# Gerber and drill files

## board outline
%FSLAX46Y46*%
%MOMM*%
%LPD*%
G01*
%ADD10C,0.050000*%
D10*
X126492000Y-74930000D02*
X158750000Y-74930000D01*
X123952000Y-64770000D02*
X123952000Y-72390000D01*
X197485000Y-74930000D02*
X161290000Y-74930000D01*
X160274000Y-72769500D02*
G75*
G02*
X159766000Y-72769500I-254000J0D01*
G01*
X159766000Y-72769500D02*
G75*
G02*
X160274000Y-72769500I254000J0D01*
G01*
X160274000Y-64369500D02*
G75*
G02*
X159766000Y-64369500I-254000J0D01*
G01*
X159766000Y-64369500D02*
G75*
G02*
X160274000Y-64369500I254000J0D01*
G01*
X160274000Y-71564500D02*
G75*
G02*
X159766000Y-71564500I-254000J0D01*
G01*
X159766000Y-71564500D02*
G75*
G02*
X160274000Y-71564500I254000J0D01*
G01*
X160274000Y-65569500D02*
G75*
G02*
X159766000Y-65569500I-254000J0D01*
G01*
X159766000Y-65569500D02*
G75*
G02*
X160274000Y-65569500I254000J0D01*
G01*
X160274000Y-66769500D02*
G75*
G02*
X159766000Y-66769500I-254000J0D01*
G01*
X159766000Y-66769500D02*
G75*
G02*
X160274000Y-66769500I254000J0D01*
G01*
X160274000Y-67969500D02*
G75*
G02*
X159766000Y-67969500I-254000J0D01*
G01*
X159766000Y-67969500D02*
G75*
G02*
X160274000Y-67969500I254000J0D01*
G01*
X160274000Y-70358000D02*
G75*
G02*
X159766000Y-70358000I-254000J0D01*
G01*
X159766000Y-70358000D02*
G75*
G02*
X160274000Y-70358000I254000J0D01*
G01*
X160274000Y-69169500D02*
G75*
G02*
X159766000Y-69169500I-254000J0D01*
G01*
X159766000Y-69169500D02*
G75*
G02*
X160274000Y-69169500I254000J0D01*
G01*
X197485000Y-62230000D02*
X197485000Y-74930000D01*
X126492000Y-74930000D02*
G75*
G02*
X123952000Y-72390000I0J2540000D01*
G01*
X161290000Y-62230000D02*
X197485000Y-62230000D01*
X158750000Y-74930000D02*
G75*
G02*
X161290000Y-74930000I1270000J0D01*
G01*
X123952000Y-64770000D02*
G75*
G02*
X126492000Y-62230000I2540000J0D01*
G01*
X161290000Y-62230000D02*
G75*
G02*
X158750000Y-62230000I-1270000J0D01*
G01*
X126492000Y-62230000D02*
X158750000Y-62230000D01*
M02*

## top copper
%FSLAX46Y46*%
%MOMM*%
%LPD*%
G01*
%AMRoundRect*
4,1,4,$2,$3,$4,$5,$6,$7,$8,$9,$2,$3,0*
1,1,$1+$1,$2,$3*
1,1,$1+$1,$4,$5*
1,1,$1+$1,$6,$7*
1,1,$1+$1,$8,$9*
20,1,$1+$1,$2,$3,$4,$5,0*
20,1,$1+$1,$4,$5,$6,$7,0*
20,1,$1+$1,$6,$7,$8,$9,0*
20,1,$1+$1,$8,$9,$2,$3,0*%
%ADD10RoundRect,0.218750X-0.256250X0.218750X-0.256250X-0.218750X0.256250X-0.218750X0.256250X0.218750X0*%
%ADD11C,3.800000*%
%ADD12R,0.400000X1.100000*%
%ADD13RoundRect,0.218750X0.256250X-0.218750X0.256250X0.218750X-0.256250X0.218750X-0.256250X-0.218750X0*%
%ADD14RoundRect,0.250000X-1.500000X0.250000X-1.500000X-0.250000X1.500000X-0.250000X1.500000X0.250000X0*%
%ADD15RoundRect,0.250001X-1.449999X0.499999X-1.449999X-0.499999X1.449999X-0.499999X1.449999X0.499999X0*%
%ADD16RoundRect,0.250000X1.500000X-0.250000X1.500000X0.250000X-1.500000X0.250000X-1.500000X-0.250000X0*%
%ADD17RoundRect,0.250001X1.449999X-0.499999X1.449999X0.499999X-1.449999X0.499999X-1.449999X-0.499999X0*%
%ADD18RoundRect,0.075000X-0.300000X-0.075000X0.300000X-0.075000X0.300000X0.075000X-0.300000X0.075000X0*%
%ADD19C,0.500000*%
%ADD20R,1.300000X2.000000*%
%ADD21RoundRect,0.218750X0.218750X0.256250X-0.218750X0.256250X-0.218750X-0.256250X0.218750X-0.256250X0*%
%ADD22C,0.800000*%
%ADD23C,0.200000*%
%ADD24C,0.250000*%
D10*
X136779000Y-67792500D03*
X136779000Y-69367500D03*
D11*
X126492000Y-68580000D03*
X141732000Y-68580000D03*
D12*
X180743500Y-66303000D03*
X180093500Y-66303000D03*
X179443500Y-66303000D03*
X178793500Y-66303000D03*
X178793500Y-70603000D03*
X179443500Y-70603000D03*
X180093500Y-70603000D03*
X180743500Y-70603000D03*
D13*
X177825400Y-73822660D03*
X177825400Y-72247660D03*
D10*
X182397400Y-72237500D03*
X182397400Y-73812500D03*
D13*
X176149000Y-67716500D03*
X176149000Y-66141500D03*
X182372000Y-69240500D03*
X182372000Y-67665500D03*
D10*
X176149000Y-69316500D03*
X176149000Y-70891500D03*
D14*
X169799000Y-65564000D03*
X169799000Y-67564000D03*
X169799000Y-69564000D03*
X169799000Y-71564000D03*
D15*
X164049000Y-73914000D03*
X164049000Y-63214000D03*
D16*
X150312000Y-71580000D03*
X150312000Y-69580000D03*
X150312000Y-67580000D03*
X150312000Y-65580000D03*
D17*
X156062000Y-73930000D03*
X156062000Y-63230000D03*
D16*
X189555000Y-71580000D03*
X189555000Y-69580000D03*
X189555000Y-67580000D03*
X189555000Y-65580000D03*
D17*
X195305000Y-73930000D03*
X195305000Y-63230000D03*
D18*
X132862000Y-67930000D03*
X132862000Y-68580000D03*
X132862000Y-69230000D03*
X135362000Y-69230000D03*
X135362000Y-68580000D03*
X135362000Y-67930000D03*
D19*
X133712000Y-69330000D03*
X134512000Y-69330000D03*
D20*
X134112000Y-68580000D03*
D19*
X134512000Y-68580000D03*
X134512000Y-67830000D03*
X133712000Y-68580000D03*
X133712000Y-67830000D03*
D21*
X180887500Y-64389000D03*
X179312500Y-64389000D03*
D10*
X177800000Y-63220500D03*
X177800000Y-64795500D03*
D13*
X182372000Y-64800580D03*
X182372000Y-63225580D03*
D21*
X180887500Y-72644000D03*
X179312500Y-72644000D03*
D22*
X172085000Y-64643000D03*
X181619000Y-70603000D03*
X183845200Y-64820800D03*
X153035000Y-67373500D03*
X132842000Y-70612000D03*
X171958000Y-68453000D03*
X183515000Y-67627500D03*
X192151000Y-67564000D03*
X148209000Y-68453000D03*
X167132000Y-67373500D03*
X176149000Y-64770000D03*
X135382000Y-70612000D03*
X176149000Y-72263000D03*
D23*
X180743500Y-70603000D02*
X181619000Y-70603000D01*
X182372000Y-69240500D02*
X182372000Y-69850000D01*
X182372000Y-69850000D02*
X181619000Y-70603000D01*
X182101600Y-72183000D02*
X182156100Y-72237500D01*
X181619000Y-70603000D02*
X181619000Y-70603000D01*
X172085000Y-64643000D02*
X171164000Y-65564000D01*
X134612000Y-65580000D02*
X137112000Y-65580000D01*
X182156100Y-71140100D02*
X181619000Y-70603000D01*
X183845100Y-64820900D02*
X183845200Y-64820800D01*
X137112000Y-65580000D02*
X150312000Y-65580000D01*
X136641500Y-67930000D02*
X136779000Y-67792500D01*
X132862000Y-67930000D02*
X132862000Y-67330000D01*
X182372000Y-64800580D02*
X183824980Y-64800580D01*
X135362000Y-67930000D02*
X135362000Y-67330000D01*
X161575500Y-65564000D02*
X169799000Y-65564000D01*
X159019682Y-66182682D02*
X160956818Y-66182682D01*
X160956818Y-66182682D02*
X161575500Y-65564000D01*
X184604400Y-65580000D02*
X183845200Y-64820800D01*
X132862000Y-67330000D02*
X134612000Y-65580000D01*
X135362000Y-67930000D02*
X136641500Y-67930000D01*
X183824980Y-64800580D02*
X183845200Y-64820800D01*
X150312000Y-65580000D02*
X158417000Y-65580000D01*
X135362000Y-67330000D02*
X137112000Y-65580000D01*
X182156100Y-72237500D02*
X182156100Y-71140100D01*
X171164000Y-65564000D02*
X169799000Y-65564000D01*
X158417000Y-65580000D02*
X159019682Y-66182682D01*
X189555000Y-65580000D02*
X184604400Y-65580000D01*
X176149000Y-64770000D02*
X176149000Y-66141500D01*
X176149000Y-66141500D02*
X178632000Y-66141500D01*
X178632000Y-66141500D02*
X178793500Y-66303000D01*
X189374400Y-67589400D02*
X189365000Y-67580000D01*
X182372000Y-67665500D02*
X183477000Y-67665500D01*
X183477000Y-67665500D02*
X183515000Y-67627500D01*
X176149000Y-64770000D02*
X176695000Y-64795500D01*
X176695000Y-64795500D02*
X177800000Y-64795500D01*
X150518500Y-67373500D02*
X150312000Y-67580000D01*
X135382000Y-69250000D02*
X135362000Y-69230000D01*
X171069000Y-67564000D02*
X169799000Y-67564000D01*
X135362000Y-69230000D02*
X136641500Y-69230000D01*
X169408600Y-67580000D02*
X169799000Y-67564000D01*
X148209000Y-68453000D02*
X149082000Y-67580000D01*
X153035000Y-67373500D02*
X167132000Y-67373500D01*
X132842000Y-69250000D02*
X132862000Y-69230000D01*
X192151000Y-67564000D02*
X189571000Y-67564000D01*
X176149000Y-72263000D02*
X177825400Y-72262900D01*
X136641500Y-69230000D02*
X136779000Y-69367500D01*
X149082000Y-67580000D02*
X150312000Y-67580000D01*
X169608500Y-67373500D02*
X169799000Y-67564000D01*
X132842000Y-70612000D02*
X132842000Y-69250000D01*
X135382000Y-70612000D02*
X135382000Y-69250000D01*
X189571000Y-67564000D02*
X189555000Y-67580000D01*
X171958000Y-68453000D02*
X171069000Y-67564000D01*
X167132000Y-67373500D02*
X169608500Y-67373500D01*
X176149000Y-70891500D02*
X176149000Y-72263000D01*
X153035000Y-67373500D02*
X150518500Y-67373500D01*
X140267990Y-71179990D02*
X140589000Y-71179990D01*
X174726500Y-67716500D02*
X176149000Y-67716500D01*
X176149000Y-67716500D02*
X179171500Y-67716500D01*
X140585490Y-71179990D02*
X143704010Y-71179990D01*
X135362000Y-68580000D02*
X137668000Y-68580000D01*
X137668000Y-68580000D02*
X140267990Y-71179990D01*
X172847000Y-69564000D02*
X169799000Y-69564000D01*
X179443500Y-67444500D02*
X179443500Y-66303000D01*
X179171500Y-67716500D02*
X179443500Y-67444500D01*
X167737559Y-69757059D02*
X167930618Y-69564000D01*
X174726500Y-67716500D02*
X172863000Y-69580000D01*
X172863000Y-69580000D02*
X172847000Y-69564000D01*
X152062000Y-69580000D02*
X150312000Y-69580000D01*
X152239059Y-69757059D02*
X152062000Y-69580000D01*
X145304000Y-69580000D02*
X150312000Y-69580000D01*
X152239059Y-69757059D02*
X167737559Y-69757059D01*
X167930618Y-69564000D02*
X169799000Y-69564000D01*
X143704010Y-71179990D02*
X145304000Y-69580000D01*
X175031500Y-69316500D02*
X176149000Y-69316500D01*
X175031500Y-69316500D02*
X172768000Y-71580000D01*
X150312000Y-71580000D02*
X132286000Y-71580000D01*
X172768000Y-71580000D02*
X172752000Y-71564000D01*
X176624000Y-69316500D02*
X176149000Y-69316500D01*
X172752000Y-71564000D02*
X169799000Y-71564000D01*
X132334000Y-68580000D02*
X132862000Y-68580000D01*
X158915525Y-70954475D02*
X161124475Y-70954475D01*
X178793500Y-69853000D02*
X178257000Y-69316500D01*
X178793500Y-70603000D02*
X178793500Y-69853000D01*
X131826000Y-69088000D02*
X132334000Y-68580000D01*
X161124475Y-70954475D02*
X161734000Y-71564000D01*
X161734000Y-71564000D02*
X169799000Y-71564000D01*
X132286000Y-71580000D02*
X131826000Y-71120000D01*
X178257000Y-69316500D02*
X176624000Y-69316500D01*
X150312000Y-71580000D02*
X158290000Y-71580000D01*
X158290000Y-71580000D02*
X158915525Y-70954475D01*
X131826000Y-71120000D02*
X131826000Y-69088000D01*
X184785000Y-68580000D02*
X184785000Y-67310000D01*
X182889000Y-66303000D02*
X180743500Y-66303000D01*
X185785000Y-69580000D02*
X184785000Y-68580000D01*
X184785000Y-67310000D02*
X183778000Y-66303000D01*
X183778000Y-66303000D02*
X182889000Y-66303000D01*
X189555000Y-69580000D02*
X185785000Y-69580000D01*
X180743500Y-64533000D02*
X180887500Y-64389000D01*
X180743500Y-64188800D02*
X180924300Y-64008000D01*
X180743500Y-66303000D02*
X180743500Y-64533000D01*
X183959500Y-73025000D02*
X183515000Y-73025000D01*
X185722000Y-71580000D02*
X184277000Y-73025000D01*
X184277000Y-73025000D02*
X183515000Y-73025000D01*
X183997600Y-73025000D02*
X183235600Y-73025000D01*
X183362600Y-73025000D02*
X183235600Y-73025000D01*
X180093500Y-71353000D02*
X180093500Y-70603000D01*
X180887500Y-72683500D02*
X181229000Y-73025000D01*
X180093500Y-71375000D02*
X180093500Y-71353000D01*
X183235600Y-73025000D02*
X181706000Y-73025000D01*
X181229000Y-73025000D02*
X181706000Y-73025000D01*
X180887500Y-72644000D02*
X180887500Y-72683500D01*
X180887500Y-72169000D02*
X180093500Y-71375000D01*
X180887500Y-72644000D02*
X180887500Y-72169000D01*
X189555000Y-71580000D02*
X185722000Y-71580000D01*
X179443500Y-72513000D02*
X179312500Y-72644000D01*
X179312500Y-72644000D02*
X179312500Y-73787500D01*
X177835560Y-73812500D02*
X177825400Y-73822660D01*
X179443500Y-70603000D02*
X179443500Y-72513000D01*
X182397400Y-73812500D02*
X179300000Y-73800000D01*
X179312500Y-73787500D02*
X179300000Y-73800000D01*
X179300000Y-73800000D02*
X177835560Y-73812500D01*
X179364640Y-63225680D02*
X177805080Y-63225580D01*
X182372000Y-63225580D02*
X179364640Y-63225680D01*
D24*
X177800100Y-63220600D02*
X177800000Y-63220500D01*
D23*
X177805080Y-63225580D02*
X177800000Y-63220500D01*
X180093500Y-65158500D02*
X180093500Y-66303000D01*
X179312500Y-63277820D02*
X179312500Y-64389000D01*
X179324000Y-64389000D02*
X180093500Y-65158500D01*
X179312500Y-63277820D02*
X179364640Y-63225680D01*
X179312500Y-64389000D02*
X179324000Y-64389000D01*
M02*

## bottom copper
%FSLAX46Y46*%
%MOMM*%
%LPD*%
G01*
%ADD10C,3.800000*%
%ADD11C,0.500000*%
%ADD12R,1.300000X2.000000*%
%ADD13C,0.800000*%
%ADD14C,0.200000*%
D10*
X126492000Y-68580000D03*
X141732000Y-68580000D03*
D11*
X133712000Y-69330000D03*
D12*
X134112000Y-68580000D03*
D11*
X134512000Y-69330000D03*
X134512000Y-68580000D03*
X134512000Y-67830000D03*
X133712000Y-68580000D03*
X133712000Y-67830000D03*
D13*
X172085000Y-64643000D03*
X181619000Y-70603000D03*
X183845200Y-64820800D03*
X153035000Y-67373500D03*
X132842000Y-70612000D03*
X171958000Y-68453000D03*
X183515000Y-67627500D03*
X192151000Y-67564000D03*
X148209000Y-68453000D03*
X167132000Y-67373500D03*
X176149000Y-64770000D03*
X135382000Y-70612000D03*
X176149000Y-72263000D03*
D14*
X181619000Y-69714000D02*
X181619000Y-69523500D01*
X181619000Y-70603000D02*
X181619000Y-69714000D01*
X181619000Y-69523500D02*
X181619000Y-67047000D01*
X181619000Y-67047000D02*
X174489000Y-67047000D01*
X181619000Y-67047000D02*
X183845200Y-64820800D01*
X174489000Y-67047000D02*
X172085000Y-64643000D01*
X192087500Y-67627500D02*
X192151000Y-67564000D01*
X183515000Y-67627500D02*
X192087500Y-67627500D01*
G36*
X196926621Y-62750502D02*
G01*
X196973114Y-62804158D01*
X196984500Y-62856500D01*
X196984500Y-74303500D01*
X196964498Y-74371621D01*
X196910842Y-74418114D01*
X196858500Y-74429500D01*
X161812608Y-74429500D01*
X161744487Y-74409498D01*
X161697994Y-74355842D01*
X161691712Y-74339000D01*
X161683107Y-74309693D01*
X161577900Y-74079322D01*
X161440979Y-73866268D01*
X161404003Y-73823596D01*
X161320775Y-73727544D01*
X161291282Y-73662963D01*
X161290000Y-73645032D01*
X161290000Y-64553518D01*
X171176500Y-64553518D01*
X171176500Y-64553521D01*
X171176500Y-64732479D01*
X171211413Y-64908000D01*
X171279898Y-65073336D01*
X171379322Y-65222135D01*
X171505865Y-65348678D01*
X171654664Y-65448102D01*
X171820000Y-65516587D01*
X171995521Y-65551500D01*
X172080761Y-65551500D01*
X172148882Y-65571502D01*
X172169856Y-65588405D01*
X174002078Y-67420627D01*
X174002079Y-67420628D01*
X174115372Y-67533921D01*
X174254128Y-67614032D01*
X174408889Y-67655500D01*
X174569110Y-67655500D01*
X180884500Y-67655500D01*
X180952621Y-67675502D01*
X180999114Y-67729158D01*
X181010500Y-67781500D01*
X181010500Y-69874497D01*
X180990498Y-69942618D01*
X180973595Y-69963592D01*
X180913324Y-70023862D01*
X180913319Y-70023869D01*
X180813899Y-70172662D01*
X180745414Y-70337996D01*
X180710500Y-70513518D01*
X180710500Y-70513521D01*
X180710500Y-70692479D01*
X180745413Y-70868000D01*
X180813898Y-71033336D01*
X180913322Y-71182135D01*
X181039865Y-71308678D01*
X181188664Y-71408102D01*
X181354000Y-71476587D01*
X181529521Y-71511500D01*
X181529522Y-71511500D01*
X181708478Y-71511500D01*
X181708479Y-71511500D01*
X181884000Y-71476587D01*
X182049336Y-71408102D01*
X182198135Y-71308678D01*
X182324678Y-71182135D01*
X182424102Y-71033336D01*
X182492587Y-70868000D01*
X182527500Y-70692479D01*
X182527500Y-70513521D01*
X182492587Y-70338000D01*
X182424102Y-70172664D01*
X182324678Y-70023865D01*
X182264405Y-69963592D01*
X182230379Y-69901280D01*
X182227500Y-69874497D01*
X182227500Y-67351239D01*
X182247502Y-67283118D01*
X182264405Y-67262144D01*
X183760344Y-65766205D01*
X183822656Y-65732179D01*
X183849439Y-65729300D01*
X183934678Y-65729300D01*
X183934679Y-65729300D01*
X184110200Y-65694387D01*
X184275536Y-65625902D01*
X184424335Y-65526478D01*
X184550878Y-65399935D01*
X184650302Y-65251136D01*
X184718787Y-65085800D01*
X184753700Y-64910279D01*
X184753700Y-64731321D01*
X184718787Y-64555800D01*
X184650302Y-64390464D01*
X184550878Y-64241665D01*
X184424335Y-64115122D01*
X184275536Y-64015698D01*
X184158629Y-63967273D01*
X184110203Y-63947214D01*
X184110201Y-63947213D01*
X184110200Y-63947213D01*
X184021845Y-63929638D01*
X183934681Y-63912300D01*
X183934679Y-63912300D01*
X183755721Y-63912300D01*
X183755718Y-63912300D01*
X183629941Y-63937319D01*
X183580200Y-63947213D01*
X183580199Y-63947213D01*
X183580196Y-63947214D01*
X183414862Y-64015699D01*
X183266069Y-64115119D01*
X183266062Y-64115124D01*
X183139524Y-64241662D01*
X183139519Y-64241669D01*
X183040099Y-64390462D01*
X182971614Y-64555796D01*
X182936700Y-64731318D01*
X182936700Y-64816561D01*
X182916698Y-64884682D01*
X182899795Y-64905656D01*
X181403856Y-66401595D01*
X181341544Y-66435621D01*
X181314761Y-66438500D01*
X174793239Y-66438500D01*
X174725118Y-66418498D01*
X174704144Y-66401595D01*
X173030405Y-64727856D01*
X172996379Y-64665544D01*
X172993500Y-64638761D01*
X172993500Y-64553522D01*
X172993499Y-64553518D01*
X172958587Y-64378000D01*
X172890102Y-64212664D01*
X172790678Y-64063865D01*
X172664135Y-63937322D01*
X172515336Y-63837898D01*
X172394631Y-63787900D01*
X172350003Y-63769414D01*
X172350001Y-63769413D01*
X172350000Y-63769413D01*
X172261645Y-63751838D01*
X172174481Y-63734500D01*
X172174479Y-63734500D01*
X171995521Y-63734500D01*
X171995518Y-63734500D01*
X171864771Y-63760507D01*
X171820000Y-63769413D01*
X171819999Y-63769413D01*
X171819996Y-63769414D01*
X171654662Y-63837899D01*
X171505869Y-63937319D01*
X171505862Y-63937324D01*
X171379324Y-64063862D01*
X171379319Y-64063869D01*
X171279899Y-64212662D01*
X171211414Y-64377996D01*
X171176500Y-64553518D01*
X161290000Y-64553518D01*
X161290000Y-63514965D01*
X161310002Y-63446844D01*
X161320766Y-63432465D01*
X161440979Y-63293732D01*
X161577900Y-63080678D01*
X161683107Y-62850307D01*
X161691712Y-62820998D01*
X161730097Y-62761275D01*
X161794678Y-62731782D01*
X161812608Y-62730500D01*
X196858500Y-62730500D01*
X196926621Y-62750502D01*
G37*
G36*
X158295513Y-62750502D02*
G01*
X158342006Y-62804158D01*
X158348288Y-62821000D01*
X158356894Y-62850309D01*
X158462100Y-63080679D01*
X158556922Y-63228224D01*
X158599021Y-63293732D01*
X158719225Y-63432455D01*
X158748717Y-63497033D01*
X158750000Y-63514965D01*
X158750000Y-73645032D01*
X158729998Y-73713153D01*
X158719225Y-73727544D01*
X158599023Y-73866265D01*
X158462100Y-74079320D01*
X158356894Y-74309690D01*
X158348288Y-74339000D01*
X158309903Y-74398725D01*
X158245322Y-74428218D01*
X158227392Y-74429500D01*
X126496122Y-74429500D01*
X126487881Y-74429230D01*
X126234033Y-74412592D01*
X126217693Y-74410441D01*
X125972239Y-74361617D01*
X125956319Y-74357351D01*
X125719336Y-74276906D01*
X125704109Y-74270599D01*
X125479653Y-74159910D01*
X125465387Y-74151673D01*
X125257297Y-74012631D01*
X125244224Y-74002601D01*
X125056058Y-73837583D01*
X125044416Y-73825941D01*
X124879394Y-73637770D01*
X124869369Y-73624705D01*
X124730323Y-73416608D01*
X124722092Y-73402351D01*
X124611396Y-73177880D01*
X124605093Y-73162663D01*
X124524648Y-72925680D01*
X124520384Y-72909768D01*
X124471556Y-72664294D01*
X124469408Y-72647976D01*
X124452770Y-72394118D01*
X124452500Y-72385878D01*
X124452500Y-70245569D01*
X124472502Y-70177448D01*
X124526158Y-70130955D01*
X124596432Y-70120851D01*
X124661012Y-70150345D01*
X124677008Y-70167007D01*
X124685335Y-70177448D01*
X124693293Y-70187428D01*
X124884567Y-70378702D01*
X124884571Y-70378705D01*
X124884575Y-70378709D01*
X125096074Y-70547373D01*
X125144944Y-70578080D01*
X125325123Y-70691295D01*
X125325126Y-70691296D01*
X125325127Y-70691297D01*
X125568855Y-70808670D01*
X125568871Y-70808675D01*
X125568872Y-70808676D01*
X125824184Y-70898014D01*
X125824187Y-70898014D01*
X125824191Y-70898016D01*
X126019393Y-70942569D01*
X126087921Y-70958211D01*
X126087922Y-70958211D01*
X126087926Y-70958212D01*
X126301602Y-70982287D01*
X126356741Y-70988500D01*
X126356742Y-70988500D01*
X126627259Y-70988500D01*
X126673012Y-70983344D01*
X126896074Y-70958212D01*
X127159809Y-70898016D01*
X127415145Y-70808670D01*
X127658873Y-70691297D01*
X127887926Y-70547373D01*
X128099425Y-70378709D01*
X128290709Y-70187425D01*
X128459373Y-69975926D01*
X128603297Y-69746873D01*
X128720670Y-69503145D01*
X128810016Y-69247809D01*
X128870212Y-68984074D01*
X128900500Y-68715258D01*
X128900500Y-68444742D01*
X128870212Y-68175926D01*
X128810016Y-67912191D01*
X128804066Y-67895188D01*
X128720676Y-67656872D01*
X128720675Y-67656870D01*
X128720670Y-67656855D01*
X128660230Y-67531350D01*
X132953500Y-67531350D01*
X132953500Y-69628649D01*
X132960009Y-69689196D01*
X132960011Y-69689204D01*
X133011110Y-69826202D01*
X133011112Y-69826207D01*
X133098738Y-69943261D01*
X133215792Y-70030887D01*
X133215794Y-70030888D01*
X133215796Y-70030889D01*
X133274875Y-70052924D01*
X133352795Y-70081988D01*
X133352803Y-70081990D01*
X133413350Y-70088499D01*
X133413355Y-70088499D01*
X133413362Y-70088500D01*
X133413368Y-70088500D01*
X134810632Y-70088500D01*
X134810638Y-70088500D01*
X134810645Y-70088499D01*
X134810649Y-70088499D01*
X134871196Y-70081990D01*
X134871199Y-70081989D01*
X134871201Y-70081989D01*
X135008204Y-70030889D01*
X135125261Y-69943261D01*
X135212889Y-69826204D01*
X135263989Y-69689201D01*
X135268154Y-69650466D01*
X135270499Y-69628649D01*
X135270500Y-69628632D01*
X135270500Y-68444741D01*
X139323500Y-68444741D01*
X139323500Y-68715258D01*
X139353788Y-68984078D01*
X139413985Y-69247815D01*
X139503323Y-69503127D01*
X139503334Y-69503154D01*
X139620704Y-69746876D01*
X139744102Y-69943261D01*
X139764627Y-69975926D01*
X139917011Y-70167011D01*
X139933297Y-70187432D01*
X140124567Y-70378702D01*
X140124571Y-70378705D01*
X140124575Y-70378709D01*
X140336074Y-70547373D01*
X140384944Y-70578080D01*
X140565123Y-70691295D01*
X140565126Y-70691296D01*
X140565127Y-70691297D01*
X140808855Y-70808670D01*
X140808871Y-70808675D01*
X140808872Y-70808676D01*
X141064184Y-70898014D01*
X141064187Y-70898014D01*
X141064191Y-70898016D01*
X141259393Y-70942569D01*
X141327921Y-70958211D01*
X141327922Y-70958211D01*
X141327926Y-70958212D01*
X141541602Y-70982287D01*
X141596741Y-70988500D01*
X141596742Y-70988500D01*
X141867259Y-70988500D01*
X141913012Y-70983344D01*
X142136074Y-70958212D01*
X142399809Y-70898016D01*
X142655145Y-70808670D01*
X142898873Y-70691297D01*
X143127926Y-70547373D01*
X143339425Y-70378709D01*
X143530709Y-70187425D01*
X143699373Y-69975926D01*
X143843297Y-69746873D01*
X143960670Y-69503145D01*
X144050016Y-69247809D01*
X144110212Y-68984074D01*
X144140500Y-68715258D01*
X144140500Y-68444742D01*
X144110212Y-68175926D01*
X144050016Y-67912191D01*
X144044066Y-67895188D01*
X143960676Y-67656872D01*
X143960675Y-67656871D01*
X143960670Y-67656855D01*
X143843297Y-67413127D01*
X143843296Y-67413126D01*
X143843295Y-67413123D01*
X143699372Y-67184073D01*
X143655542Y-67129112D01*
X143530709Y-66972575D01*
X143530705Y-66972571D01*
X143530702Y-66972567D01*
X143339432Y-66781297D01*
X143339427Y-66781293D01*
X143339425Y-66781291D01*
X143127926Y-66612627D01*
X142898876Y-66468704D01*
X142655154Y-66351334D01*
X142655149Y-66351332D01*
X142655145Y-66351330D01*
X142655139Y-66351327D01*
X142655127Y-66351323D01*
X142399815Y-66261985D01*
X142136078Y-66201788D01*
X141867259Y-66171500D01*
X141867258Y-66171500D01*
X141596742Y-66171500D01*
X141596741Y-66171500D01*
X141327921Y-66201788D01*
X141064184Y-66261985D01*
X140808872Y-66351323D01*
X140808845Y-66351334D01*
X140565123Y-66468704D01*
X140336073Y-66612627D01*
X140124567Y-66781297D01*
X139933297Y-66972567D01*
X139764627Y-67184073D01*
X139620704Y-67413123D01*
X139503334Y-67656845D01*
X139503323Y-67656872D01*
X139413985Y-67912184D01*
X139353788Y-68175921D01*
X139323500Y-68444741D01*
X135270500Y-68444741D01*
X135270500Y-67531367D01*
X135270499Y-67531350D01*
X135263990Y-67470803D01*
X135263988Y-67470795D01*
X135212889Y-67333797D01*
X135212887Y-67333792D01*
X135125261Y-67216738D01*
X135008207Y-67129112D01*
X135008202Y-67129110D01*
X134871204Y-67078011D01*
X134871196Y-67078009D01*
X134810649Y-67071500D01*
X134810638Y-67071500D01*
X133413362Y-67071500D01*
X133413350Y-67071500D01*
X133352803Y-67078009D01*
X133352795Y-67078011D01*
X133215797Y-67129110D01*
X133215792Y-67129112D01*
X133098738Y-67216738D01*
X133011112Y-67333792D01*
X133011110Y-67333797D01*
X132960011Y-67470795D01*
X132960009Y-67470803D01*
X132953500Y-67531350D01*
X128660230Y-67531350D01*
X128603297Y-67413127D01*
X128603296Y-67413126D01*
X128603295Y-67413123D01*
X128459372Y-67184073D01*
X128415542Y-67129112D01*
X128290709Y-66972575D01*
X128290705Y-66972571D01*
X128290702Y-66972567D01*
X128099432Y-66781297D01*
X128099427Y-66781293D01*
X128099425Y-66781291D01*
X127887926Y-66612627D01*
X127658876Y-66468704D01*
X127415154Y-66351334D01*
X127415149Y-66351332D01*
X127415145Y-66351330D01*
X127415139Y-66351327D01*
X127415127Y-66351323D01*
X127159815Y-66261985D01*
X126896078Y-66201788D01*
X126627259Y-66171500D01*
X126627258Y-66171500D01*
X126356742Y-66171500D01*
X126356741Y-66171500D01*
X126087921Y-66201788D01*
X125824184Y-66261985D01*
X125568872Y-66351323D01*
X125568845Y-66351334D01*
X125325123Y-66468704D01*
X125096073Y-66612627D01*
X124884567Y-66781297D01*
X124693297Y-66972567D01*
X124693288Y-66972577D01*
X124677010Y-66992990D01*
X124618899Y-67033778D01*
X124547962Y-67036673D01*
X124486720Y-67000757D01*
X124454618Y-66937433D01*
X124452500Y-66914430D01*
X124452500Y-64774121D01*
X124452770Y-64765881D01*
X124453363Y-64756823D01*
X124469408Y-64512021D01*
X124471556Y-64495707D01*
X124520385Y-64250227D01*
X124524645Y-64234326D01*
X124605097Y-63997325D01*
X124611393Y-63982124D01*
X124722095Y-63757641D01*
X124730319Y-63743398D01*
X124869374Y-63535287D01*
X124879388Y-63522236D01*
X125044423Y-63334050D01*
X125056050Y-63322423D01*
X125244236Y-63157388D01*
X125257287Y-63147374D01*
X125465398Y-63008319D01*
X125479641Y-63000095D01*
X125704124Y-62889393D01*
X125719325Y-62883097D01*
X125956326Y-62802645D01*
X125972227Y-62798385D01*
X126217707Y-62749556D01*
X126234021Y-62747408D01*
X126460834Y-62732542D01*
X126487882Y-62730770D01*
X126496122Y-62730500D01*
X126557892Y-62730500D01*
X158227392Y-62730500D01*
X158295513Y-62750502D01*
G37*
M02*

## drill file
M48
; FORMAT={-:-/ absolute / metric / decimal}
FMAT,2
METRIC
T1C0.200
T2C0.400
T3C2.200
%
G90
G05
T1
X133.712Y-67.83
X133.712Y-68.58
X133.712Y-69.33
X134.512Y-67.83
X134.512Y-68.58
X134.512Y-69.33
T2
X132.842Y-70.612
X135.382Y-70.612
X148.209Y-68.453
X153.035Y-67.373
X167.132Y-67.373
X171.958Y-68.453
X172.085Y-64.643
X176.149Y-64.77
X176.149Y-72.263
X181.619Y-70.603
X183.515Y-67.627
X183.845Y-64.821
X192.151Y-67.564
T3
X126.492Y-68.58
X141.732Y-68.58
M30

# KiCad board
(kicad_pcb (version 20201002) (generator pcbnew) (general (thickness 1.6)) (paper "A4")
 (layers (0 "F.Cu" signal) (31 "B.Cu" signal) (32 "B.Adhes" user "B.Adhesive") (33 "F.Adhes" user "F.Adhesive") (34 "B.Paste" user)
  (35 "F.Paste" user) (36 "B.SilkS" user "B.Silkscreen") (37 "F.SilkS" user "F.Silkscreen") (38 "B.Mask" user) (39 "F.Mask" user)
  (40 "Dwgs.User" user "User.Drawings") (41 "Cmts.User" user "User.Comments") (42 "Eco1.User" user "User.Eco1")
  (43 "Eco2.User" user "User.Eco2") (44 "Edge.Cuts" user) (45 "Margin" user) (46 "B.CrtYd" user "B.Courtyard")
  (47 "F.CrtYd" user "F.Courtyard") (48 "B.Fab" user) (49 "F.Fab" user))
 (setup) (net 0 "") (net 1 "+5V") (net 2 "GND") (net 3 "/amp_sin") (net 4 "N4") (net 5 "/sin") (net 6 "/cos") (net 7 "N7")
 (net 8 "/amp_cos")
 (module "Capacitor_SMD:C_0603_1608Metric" (layer "F.Cu") (at 136.779 68.58 -90)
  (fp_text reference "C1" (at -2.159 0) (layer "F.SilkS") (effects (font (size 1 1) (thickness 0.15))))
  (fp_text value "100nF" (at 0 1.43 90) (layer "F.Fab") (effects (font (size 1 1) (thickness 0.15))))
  (pad "1" smd roundrect (at -0.7875 0 270) (size 0.875 0.95) (layers "F.Cu" "F.Paste" "F.Mask") (roundrect_rratio 0.25) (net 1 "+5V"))
  (pad "2" smd roundrect (at 0.7875 0 270) (size 0.875 0.95) (layers "F.Cu" "F.Paste" "F.Mask") (roundrect_rratio 0.25) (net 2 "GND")))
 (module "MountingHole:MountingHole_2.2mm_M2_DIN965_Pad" (layer "F.Cu") (at 126.492 68.58)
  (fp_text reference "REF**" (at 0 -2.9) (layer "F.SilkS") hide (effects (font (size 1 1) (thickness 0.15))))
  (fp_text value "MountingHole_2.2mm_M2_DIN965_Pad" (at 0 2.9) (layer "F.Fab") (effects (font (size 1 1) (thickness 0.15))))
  (pad "1" thru_hole circle (at 0 0) (size 3.8 3.8) (drill 2.2) (layers *.Cu *.Mask)))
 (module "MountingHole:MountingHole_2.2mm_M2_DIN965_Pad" (layer "F.Cu") (at 141.732 68.58)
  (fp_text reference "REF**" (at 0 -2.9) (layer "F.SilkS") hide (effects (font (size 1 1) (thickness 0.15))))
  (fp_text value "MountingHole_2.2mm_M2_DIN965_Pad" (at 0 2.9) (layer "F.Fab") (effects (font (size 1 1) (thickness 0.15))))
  (pad "1" thru_hole circle (at 0 0) (size 3.8 3.8) (drill 2.2) (layers *.Cu *.Mask)))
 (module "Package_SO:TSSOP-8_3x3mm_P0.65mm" (layer "F.Cu") (at 179.7685 68.453 -90)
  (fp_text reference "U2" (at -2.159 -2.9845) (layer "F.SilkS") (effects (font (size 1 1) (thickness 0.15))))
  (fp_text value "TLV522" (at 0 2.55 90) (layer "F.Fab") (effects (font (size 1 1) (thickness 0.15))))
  (pad "1" smd rect (at -2.15 -0.975 270) (size 1.1 0.4) (layers "F.Cu" "F.Paste" "F.Mask") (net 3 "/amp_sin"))
  (pad "2" smd rect (at -2.15 -0.325 270) (size 1.1 0.4) (layers "F.Cu" "F.Paste" "F.Mask") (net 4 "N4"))
  (pad "3" smd rect (at -2.15 0.325 270) (size 1.1 0.4) (layers "F.Cu" "F.Paste" "F.Mask") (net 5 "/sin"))
  (pad "4" smd rect (at -2.15 0.975 270) (size 1.1 0.4) (layers "F.Cu" "F.Paste" "F.Mask") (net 2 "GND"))
  (pad "5" smd rect (at 2.15 0.975 270) (size 1.1 0.4) (layers "F.Cu" "F.Paste" "F.Mask") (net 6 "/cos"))
  (pad "6" smd rect (at 2.15 0.325 270) (size 1.1 0.4) (layers "F.Cu" "F.Paste" "F.Mask") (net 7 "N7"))
  (pad "7" smd rect (at 2.15 -0.325 270) (size 1.1 0.4) (layers "F.Cu" "F.Paste" "F.Mask") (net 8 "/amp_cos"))
  (pad "8" smd rect (at 2.15 -0.975 270) (size 1.1 0.4) (layers "F.Cu" "F.Paste" "F.Mask") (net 1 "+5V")))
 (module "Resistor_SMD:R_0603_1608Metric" (layer "F.Cu") (at 177.8254 73.03516 90)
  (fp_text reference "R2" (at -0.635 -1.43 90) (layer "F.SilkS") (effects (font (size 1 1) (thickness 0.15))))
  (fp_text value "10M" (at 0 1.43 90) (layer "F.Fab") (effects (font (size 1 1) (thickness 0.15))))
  (pad "1" smd roundrect (at -0.7875 0 90) (size 0.875 0.95) (layers "F.Cu" "F.Paste" "F.Mask") (roundrect_rratio 0.25) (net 7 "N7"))
  (pad "2" smd roundrect (at 0.7875 0 90) (size 0.875 0.95) (layers "F.Cu" "F.Paste" "F.Mask") (roundrect_rratio 0.25) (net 2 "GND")))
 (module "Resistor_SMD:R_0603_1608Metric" (layer "F.Cu") (at 182.3974 73.025 -90)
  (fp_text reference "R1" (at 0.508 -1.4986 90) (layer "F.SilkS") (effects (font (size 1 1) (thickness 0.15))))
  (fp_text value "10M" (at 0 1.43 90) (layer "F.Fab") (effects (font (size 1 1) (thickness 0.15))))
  (pad "1" smd roundrect (at -0.7875 0 270) (size 0.875 0.95) (layers "F.Cu" "F.Paste" "F.Mask") (roundrect_rratio 0.25) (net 1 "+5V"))
  (pad "2" smd roundrect (at 0.7875 0 270) (size 0.875 0.95) (layers "F.Cu" "F.Paste" "F.Mask") (roundrect_rratio 0.25) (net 7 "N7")))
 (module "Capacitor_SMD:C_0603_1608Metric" (layer "F.Cu") (at 176.149 66.929 90)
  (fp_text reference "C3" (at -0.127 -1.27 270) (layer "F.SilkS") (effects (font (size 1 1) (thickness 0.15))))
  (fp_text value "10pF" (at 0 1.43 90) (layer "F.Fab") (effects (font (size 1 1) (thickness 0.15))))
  (pad "1" smd roundrect (at -0.7875 0 90) (size 0.875 0.95) (layers "F.Cu" "F.Paste" "F.Mask") (roundrect_rratio 0.25) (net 5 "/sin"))
  (pad "2" smd roundrect (at 0.7875 0 90) (size 0.875 0.95) (layers "F.Cu" "F.Paste" "F.Mask") (roundrect_rratio 0.25) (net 2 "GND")))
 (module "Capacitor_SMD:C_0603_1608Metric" (layer "F.Cu") (at 182.372 68.453 90)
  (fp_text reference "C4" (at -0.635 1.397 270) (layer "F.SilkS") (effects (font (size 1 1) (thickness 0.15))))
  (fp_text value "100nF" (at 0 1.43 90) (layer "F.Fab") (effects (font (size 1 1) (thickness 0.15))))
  (pad "1" smd roundrect (at -0.7875 0 90) (size 0.875 0.95) (layers "F.Cu" "F.Paste" "F.Mask") (roundrect_rratio 0.25) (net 1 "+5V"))
  (pad "2" smd roundrect (at 0.7875 0 90) (size 0.875 0.95) (layers "F.Cu" "F.Paste" "F.Mask") (roundrect_rratio 0.25) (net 2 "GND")))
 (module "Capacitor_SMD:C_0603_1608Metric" (layer "F.Cu") (at 176.149 70.104 -90)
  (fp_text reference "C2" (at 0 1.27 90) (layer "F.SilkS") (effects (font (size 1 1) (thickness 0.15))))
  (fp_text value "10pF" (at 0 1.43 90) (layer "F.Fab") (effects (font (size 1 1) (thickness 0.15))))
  (pad "1" smd roundrect (at -0.7875 0 270) (size 0.875 0.95) (layers "F.Cu" "F.Paste" "F.Mask") (roundrect_rratio 0.25) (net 6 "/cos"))
  (pad "2" smd roundrect (at 0.7875 0 270) (size 0.875 0.95) (layers "F.Cu" "F.Paste" "F.Mask") (roundrect_rratio 0.25) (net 2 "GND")))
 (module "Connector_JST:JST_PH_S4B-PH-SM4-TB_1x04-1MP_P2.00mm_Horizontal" (layer "F.Cu") (at 166.949 68.564 -90)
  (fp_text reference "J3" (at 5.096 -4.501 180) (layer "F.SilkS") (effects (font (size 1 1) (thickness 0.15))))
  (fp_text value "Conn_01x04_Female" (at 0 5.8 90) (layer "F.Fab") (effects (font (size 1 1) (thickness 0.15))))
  (pad "1" smd roundrect (at -3 -2.85 270) (size 1 3.5) (layers "F.Cu" "F.Paste" "F.Mask") (roundrect_rratio 0.25) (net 1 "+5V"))
  (pad "2" smd roundrect (at -1 -2.85 270) (size 1 3.5) (layers "F.Cu" "F.Paste" "F.Mask") (roundrect_rratio 0.25) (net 2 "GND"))
  (pad "3" smd roundrect (at 1 -2.85 270) (size 1 3.5) (layers "F.Cu" "F.Paste" "F.Mask") (roundrect_rratio 0.25) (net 5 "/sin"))
  (pad "4" smd roundrect (at 3 -2.85 270) (size 1 3.5) (layers "F.Cu" "F.Paste" "F.Mask") (roundrect_rratio 0.25) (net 6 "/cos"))
  (pad "MP" smd roundrect (at 5.35 2.9 270) (size 1.5 3.4) (layers "F.Cu" "F.Paste" "F.Mask") (roundrect_rratio 0.166667))
  (pad "MP" smd roundrect (at -5.35 2.9 270) (size 1.5 3.4) (layers "F.Cu" "F.Paste" "F.Mask") (roundrect_rratio 0.166667)))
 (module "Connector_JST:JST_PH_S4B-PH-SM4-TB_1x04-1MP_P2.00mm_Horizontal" (layer "F.Cu") (at 153.162 68.58 90)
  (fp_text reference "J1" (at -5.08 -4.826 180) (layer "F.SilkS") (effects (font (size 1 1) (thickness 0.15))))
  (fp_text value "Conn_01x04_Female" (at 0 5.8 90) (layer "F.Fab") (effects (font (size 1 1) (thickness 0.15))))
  (pad "1" smd roundrect (at -3 -2.85 90) (size 1 3.5) (layers "F.Cu" "F.Paste" "F.Mask") (roundrect_rratio 0.25) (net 6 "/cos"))
  (pad "2" smd roundrect (at -1 -2.85 90) (size 1 3.5) (layers "F.Cu" "F.Paste" "F.Mask") (roundrect_rratio 0.25) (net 5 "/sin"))
  (pad "3" smd roundrect (at 1 -2.85 90) (size 1 3.5) (layers "F.Cu" "F.Paste" "F.Mask") (roundrect_rratio 0.25) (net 2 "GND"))
  (pad "4" smd roundrect (at 3 -2.85 90) (size 1 3.5) (layers "F.Cu" "F.Paste" "F.Mask") (roundrect_rratio 0.25) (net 1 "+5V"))
  (pad "MP" smd roundrect (at -5.35 2.9 90) (size 1.5 3.4) (layers "F.Cu" "F.Paste" "F.Mask") (roundrect_rratio 0.166667))
  (pad "MP" smd roundrect (at 5.35 2.9 90) (size 1.5 3.4) (layers "F.Cu" "F.Paste" "F.Mask") (roundrect_rratio 0.166667)))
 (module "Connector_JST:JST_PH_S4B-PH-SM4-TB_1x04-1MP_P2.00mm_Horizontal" (layer "F.Cu") (at 192.405 68.58 90)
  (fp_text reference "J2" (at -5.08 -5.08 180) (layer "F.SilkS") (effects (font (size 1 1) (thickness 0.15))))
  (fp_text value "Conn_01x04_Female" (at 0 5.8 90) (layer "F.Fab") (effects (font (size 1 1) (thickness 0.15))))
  (pad "1" smd roundrect (at -3 -2.85 90) (size 1 3.5) (layers "F.Cu" "F.Paste" "F.Mask") (roundrect_rratio 0.25) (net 8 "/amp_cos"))
  (pad "2" smd roundrect (at -1 -2.85 90) (size 1 3.5) (layers "F.Cu" "F.Paste" "F.Mask") (roundrect_rratio 0.25) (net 3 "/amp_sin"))
  (pad "3" smd roundrect (at 1 -2.85 90) (size 1 3.5) (layers "F.Cu" "F.Paste" "F.Mask") (roundrect_rratio 0.25) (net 2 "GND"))
  (pad "4" smd roundrect (at 3 -2.85 90) (size 1 3.5) (layers "F.Cu" "F.Paste" "F.Mask") (roundrect_rratio 0.25) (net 1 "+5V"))
  (pad "MP" smd roundrect (at -5.35 2.9 90) (size 1.5 3.4) (layers "F.Cu" "F.Paste" "F.Mask") (roundrect_rratio 0.166667))
  (pad "MP" smd roundrect (at 5.35 2.9 90) (size 1.5 3.4) (layers "F.Cu" "F.Paste" "F.Mask") (roundrect_rratio 0.166667)))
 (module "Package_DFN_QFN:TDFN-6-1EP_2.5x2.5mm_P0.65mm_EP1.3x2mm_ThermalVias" (layer "F.Cu") (at 134.112 68.58)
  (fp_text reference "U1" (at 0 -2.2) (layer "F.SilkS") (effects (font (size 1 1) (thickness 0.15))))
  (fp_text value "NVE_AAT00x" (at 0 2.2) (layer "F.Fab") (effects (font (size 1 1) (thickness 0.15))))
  (pad "" smd roundrect (at 0.325 -0.5) (size 0.56 0.87) (layers "F.Paste") (roundrect_rratio 0.25))
  (pad "" smd roundrect (at 0.325 0.5) (size 0.56 0.87) (layers "F.Paste") (roundrect_rratio 0.25))
  (pad "" smd roundrect (at -0.325 0.5) (size 0.56 0.87) (layers "F.Paste") (roundrect_rratio 0.25))
  (pad "" smd roundrect (at -0.325 -0.5) (size 0.56 0.87) (layers "F.Paste") (roundrect_rratio 0.25))
  (pad "1" smd roundrect (at -1.25 -0.65) (size 0.75 0.3) (layers "F.Cu" "F.Paste" "F.Mask") (roundrect_rratio 0.25) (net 1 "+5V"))
  (pad "2" smd roundrect (at -1.25 0) (size 0.75 0.3) (layers "F.Cu" "F.Paste" "F.Mask") (roundrect_rratio 0.25) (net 6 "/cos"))
  (pad "3" smd roundrect (at -1.25 0.65) (size 0.75 0.3) (layers "F.Cu" "F.Paste" "F.Mask") (roundrect_rratio 0.25) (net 2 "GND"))
  (pad "4" smd roundrect (at 1.25 0.65) (size 0.75 0.3) (layers "F.Cu" "F.Paste" "F.Mask") (roundrect_rratio 0.25) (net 2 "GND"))
  (pad "5" smd roundrect (at 1.25 0) (size 0.75 0.3) (layers "F.Cu" "F.Paste" "F.Mask") (roundrect_rratio 0.25) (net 5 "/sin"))
  (pad "6" smd roundrect (at 1.25 -0.65) (size 0.75 0.3) (layers "F.Cu" "F.Paste" "F.Mask") (roundrect_rratio 0.25) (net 1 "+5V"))
  (pad "7" thru_hole circle (at -0.4 0.75) (size 0.5 0.5) (drill 0.2) (layers *.Cu))
  (pad "7" smd rect (at 0 0) (size 1.3 2) (layers "B.Cu"))
  (pad "7" thru_hole circle (at 0.4 0.75) (size 0.5 0.5) (drill 0.2) (layers *.Cu))
  (pad "7" smd rect (at 0 0) (size 1.3 2) (layers "F.Cu" "F.Mask"))
  (pad "7" thru_hole circle (at 0.4 0) (size 0.5 0.5) (drill 0.2) (layers *.Cu))
  (pad "7" thru_hole circle (at 0.4 -0.75) (size 0.5 0.5) (drill 0.2) (layers *.Cu))
  (pad "7" thru_hole circle (at -0.4 0) (size 0.5 0.5) (drill 0.2) (layers *.Cu))
  (pad "7" thru_hole circle (at -0.4 -0.75) (size 0.5 0.5) (drill 0.2) (layers *.Cu)))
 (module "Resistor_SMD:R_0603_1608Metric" (layer "F.Cu") (at 180.1 64.389 180)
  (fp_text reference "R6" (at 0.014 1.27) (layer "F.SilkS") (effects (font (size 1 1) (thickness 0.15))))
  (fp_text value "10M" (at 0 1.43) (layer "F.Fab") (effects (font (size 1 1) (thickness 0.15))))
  (pad "1" smd roundrect (at -0.7875 0 180) (size 0.875 0.95) (layers "F.Cu" "F.Paste" "F.Mask") (roundrect_rratio 0.25) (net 3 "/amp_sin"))
  (pad "2" smd roundrect (at 0.7875 0 180) (size 0.875 0.95) (layers "F.Cu" "F.Paste" "F.Mask") (roundrect_rratio 0.25) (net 4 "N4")))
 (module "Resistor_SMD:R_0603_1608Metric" (layer "F.Cu") (at 177.8 64.008 -90)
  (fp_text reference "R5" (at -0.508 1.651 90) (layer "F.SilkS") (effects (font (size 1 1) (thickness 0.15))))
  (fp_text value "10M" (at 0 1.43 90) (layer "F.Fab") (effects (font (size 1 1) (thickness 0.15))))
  (pad "1" smd roundrect (at -0.7875 0 270) (size 0.875 0.95) (layers "F.Cu" "F.Paste" "F.Mask") (roundrect_rratio 0.25) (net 4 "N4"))
  (pad "2" smd roundrect (at 0.7875 0 270) (size 0.875 0.95) (layers "F.Cu" "F.Paste" "F.Mask") (roundrect_rratio 0.25) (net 2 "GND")))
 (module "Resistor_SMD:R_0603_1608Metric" (layer "F.Cu") (at 182.372 64.01308 90)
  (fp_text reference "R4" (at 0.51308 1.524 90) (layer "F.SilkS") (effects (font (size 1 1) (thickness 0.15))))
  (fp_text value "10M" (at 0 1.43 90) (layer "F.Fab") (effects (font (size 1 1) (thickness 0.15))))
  (pad "1" smd roundrect (at -0.7875 0 90) (size 0.875 0.95) (layers "F.Cu" "F.Paste" "F.Mask") (roundrect_rratio 0.25) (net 1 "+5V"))
  (pad "2" smd roundrect (at 0.7875 0 90) (size 0.875 0.95) (layers "F.Cu" "F.Paste" "F.Mask") (roundrect_rratio 0.25) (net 4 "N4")))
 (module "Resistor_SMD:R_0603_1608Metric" (layer "F.Cu") (at 180.1 72.644 180)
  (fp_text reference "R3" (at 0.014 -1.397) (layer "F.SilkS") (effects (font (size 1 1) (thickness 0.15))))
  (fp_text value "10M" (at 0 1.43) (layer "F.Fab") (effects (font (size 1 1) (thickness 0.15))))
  (pad "1" smd roundrect (at -0.7875 0 180) (size 0.875 0.95) (layers "F.Cu" "F.Paste" "F.Mask") (roundrect_rratio 0.25) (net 8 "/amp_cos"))
  (pad "2" smd roundrect (at 0.7875 0 180) (size 0.875 0.95) (layers "F.Cu" "F.Paste" "F.Mask") (roundrect_rratio 0.25) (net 7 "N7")))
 (gr_line (start 126.492 74.93) (end 158.75 74.93) (layer "Edge.Cuts") (width 0.05))
 (gr_line (start 123.952 64.77) (end 123.952 72.39) (layer "Edge.Cuts") (width 0.05))
 (gr_line (start 197.485 74.93) (end 161.29 74.93) (layer "Edge.Cuts") (width 0.05))
 (gr_circle (center 160.02 72.7695) (end 160.02 73.0235) (layer "Edge.Cuts") (width 0.05))
 (gr_circle (center 160.02 64.3695) (end 160.02 64.6235) (layer "Edge.Cuts") (width 0.05))
 (gr_circle (center 160.02 71.5645) (end 160.02 71.8185) (layer "Edge.Cuts") (width 0.05))
 (gr_circle (center 160.02 65.5695) (end 160.02 65.8235) (layer "Edge.Cuts") (width 0.05))
 (gr_circle (center 160.02 66.7695) (end 160.02 67.0235) (layer "Edge.Cuts") (width 0.05))
 (gr_circle (center 160.02 67.9695) (end 160.02 68.2235) (layer "Edge.Cuts") (width 0.05))
 (gr_circle (center 160.02 70.358) (end 160.02 70.612) (layer "Edge.Cuts") (width 0.05))
 (gr_circle (center 160.02 69.1695) (end 160.02 69.4235) (layer "Edge.Cuts") (width 0.05))
 (gr_line (start 197.485 62.23) (end 197.485 74.93) (layer "Edge.Cuts") (width 0.05))
 (gr_arc (start 126.492 72.39) (end 123.952 72.39) (angle -90) (layer "Edge.Cuts") (width 0.05))
 (gr_line (start 161.29 62.23) (end 197.485 62.23) (layer "Edge.Cuts") (width 0.05))
 (gr_arc (start 160.02 74.93) (end 161.29 74.93) (angle -180) (layer "Edge.Cuts") (width 0.05))
 (gr_arc (start 126.492 64.77) (end 126.492 62.23) (angle -90) (layer "Edge.Cuts") (width 0.05))
 (gr_arc (start 160.02 62.23) (end 158.75 62.23) (angle -180) (layer "Edge.Cuts") (width 0.05))
 (gr_line (start 126.492 62.23) (end 158.75 62.23) (layer "Edge.Cuts") (width 0.05))
 (segment (start 180.7435 70.603) (end 181.619 70.603) (width 0.2) (layer "F.Cu") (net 1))
 (segment (start 182.372 69.2405) (end 182.372 69.85) (width 0.2) (layer "F.Cu") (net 1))
 (segment (start 182.372 69.85) (end 181.619 70.603) (width 0.2) (layer "F.Cu") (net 1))
 (segment (start 182.1016 72.183) (end 182.1561 72.2375) (width 0.2) (layer "F.Cu") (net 1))
 (segment (start 181.619 70.603) (end 181.619 70.603) (width 0.2) (layer "F.Cu") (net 1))
 (segment (start 172.085 64.643) (end 171.164 65.564) (width 0.2) (layer "F.Cu") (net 1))
 (segment (start 134.612 65.58) (end 137.112 65.58) (width 0.2) (layer "F.Cu") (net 1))
 (segment (start 182.1561 71.1401) (end 181.619 70.603) (width 0.2) (layer "F.Cu") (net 1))
 (segment (start 183.8451 64.8209) (end 183.8452 64.8208) (width 0.2) (layer "F.Cu") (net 1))
 (segment (start 137.112 65.58) (end 150.312 65.58) (width 0.2) (layer "F.Cu") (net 1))
 (segment (start 136.6415 67.93) (end 136.779 67.7925) (width 0.2) (layer "F.Cu") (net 1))
 (segment (start 132.862 67.93) (end 132.862 67.33) (width 0.2) (layer "F.Cu") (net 1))
 (segment (start 182.372 64.80058) (end 183.82498 64.80058) (width 0.2) (layer "F.Cu") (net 1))
 (segment (start 135.362 67.93) (end 135.362 67.33) (width 0.2) (layer "F.Cu") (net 1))
 (segment (start 161.5755 65.564) (end 169.799 65.564) (width 0.2) (layer "F.Cu") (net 1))
 (segment (start 159.019682 66.182682) (end 160.956818 66.182682) (width 0.2) (layer "F.Cu") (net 1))
 (segment (start 160.956818 66.182682) (end 161.5755 65.564) (width 0.2) (layer "F.Cu") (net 1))
 (segment (start 184.6044 65.58) (end 183.8452 64.8208) (width 0.2) (layer "F.Cu") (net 1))
 (segment (start 132.862 67.33) (end 134.612 65.58) (width 0.2) (layer "F.Cu") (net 1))
 (segment (start 135.362 67.93) (end 136.6415 67.93) (width 0.2) (layer "F.Cu") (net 1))
 (segment (start 183.82498 64.80058) (end 183.8452 64.8208) (width 0.2) (layer "F.Cu") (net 1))
 (segment (start 150.312 65.58) (end 158.417 65.58) (width 0.2) (layer "F.Cu") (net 1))
 (segment (start 135.362 67.33) (end 137.112 65.58) (width 0.2) (layer "F.Cu") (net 1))
 (segment (start 182.1561 72.2375) (end 182.1561 71.1401) (width 0.2) (layer "F.Cu") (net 1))
 (segment (start 171.164 65.564) (end 169.799 65.564) (width 0.2) (layer "F.Cu") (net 1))
 (segment (start 158.417 65.58) (end 159.019682 66.182682) (width 0.2) (layer "F.Cu") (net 1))
 (segment (start 189.555 65.58) (end 184.6044 65.58) (width 0.2) (layer "F.Cu") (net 1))
 (via (at 172.085 64.643) (size 0.8) (drill 0.4) (layers "F.Cu" "B.Cu") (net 1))
 (via (at 181.619 70.603) (size 0.8) (drill 0.4) (layers "F.Cu" "B.Cu") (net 1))
 (via (at 183.8452 64.8208) (size 0.8) (drill 0.4) (layers "F.Cu" "B.Cu") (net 1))
 (segment (start 181.619 69.714) (end 181.619 69.5235) (width 0.2) (layer "B.Cu") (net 1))
 (segment (start 181.619 70.603) (end 181.619 69.714) (width 0.2) (layer "B.Cu") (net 1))
 (segment (start 181.619 69.5235) (end 181.619 67.047) (width 0.2) (layer "B.Cu") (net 1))
 (segment (start 181.619 67.047) (end 174.489 67.047) (width 0.2) (layer "B.Cu") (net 1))
 (segment (start 181.619 67.047) (end 183.8452 64.8208) (width 0.2) (layer "B.Cu") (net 1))
 (segment (start 174.489 67.047) (end 172.085 64.643) (width 0.2) (layer "B.Cu") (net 1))
 (segment (start 176.149 64.77) (end 176.149 66.1415) (width 0.2) (layer "F.Cu") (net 2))
 (segment (start 176.149 66.1415) (end 178.632 66.1415) (width 0.2) (layer "F.Cu") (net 2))
 (segment (start 178.632 66.1415) (end 178.7935 66.303) (width 0.2) (layer "F.Cu") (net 2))
 (segment (start 189.3744 67.5894) (end 189.365 67.58) (width 0.2) (layer "F.Cu") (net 2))
 (segment (start 182.372 67.6655) (end 183.477 67.6655) (width 0.2) (layer "F.Cu") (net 2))
 (segment (start 183.477 67.6655) (end 183.515 67.6275) (width 0.2) (layer "F.Cu") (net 2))
 (segment (start 176.149 64.77) (end 176.695 64.7955) (width 0.2) (layer "F.Cu") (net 2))
 (segment (start 176.695 64.7955) (end 177.8 64.7955) (width 0.2) (layer "F.Cu") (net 2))
 (segment (start 150.5185 67.3735) (end 150.312 67.58) (width 0.2) (layer "F.Cu") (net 2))
 (segment (start 135.382 69.25) (end 135.362 69.23) (width 0.2) (layer "F.Cu") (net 2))
 (segment (start 171.069 67.564) (end 169.799 67.564) (width 0.2) (layer "F.Cu") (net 2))
 (segment (start 135.362 69.23) (end 136.6415 69.23) (width 0.2) (layer "F.Cu") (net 2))
 (segment (start 169.4086 67.58) (end 169.799 67.564) (width 0.2) (layer "F.Cu") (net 2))
 (segment (start 148.209 68.453) (end 149.082 67.58) (width 0.2) (layer "F.Cu") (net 2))
 (segment (start 153.035 67.3735) (end 167.132 67.3735) (width 0.2) (layer "F.Cu") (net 2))
 (segment (start 132.842 69.25) (end 132.862 69.23) (width 0.2) (layer "F.Cu") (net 2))
 (segment (start 192.151 67.564) (end 189.571 67.564) (width 0.2) (layer "F.Cu") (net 2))
 (segment (start 176.149 72.263) (end 177.8254 72.2629) (width 0.2) (layer "F.Cu") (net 2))
 (segment (start 136.6415 69.23) (end 136.779 69.3675) (width 0.2) (layer "F.Cu") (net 2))
 (segment (start 149.082 67.58) (end 150.312 67.58) (width 0.2) (layer "F.Cu") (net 2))
 (segment (start 169.6085 67.3735) (end 169.799 67.564) (width 0.2) (layer "F.Cu") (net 2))
 (segment (start 132.842 70.612) (end 132.842 69.25) (width 0.2) (layer "F.Cu") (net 2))
 (segment (start 135.382 70.612) (end 135.382 69.25) (width 0.2) (layer "F.Cu") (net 2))
 (segment (start 189.571 67.564) (end 189.555 67.58) (width 0.2) (layer "F.Cu") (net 2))
 (segment (start 171.958 68.453) (end 171.069 67.564) (width 0.2) (layer "F.Cu") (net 2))
 (segment (start 167.132 67.3735) (end 169.6085 67.3735) (width 0.2) (layer "F.Cu") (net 2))
 (segment (start 176.149 70.8915) (end 176.149 72.263) (width 0.2) (layer "F.Cu") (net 2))
 (segment (start 153.035 67.3735) (end 150.5185 67.3735) (width 0.2) (layer "F.Cu") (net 2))
 (via (at 153.035 67.3735) (size 0.8) (drill 0.4) (layers "F.Cu" "B.Cu") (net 2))
 (via (at 132.842 70.612) (size 0.8) (drill 0.4) (layers "F.Cu" "B.Cu") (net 2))
 (via (at 171.958 68.453) (size 0.8) (drill 0.4) (layers "F.Cu" "B.Cu") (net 2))
 (via (at 183.515 67.6275) (size 0.8) (drill 0.4) (layers "F.Cu" "B.Cu") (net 2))
 (via (at 192.151 67.564) (size 0.8) (drill 0.4) (layers "F.Cu" "B.Cu") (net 2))
 (via (at 148.209 68.453) (size 0.8) (drill 0.4) (layers "F.Cu" "B.Cu") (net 2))
 (via (at 167.132 67.3735) (size 0.8) (drill 0.4) (layers "F.Cu" "B.Cu") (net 2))
 (via (at 176.149 64.77) (size 0.8) (drill 0.4) (layers "F.Cu" "B.Cu") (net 2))
 (via (at 135.382 70.612) (size 0.8) (drill 0.4) (layers "F.Cu" "B.Cu") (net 2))
 (via (at 176.149 72.263) (size 0.8) (drill 0.4) (layers "F.Cu" "B.Cu") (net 2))
 (segment (start 192.0875 67.6275) (end 192.151 67.564) (width 0.2) (layer "B.Cu") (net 2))
 (segment (start 183.515 67.6275) (end 192.0875 67.6275) (width 0.2) (layer "B.Cu") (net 2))
 (segment (start 140.26799 71.17999) (end 140.589 71.17999) (width 0.2) (layer "F.Cu") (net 5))
 (segment (start 174.7265 67.7165) (end 176.149 67.7165) (width 0.2) (layer "F.Cu") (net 5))
 (segment (start 176.149 67.7165) (end 179.1715 67.7165) (width 0.2) (layer "F.Cu") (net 5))
 (segment (start 140.58549 71.17999) (end 143.70401 71.17999) (width 0.2) (layer "F.Cu") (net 5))
 (segment (start 135.362 68.58) (end 137.668 68.58) (width 0.2) (layer "F.Cu") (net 5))
 (segment (start 137.668 68.58) (end 140.26799 71.17999) (width 0.2) (layer "F.Cu") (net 5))
 (segment (start 172.847 69.564) (end 169.799 69.564) (width 0.2) (layer "F.Cu") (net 5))
 (segment (start 179.4435 67.4445) (end 179.4435 66.303) (width 0.2) (layer "F.Cu") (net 5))
 (segment (start 179.1715 67.7165) (end 179.4435 67.4445) (width 0.2) (layer "F.Cu") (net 5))
 (segment (start 167.737559 69.757059) (end 167.930618 69.564) (width 0.2) (layer "F.Cu") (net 5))
 (segment (start 174.7265 67.7165) (end 172.863 69.58) (width 0.2) (layer "F.Cu") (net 5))
 (segment (start 172.863 69.58) (end 172.847 69.564) (width 0.2) (layer "F.Cu") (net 5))
 (segment (start 152.062 69.58) (end 150.312 69.58) (width 0.2) (layer "F.Cu") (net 5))
 (segment (start 152.239059 69.757059) (end 152.062 69.58) (width 0.2) (layer "F.Cu") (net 5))
 (segment (start 145.304 69.58) (end 150.312 69.58) (width 0.2) (layer "F.Cu") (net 5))
 (segment (start 152.239059 69.757059) (end 167.737559 69.757059) (width 0.2) (layer "F.Cu") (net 5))
 (segment (start 167.930618 69.564) (end 169.799 69.564) (width 0.2) (layer "F.Cu") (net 5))
 (segment (start 143.70401 71.17999) (end 145.304 69.58) (width 0.2) (layer "F.Cu") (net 5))
 (segment (start 175.0315 69.3165) (end 176.149 69.3165) (width 0.2) (layer "F.Cu") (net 6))
 (segment (start 175.0315 69.3165) (end 172.768 71.58) (width 0.2) (layer "F.Cu") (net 6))
 (segment (start 150.312 71.58) (end 132.286 71.58) (width 0.2) (layer "F.Cu") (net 6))
 (segment (start 172.768 71.58) (end 172.752 71.564) (width 0.2) (layer "F.Cu") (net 6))
 (segment (start 176.624 69.3165) (end 176.149 69.3165) (width 0.2) (layer "F.Cu") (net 6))
 (segment (start 172.752 71.564) (end 169.799 71.564) (width 0.2) (layer "F.Cu") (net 6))
 (segment (start 132.334 68.58) (end 132.862 68.58) (width 0.2) (layer "F.Cu") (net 6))
 (segment (start 158.915525 70.954475) (end 161.124475 70.954475) (width 0.2) (layer "F.Cu") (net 6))
 (segment (start 178.7935 69.853) (end 178.257 69.3165) (width 0.2) (layer "F.Cu") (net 6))
 (segment (start 178.7935 70.603) (end 178.7935 69.853) (width 0.2) (layer "F.Cu") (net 6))
 (segment (start 131.826 69.088) (end 132.334 68.58) (width 0.2) (layer "F.Cu") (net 6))
 (segment (start 161.124475 70.954475) (end 161.734 71.564) (width 0.2) (layer "F.Cu") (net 6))
 (segment (start 161.734 71.564) (end 169.799 71.564) (width 0.2) (layer "F.Cu") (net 6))
 (segment (start 132.286 71.58) (end 131.826 71.12) (width 0.2) (layer "F.Cu") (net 6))
 (segment (start 178.257 69.3165) (end 176.624 69.3165) (width 0.2) (layer "F.Cu") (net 6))
 (segment (start 150.312 71.58) (end 158.29 71.58) (width 0.2) (layer "F.Cu") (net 6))
 (segment (start 158.29 71.58) (end 158.915525 70.954475) (width 0.2) (layer "F.Cu") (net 6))
 (segment (start 131.826 71.12) (end 131.826 69.088) (width 0.2) (layer "F.Cu") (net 6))
 (segment (start 184.785 68.58) (end 184.785 67.31) (width 0.2) (layer "F.Cu") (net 3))
 (segment (start 182.889 66.303) (end 180.7435 66.303) (width 0.2) (layer "F.Cu") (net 3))
 (segment (start 185.785 69.58) (end 184.785 68.58) (width 0.2) (layer "F.Cu") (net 3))
 (segment (start 184.785 67.31) (end 183.778 66.303) (width 0.2) (layer "F.Cu") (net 3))
 (segment (start 183.778 66.303) (end 182.889 66.303) (width 0.2) (layer "F.Cu") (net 3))
 (segment (start 189.555 69.58) (end 185.785 69.58) (width 0.2) (layer "F.Cu") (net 3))
 (segment (start 180.7435 64.533) (end 180.8875 64.389) (width 0.2) (layer "F.Cu") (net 3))
 (segment (start 180.7435 64.1888) (end 180.9243 64.008) (width 0.2) (layer "F.Cu") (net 3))
 (segment (start 180.7435 66.303) (end 180.7435 64.533) (width 0.2) (layer "F.Cu") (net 3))
 (segment (start 183.9595 73.025) (end 183.515 73.025) (width 0.2) (layer "F.Cu") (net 8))
 (segment (start 185.722 71.58) (end 184.277 73.025) (width 0.2) (layer "F.Cu") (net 8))
 (segment (start 184.277 73.025) (end 183.515 73.025) (width 0.2) (layer "F.Cu") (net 8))
 (segment (start 183.9976 73.025) (end 183.2356 73.025) (width 0.2) (layer "F.Cu") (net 8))
 (segment (start 183.3626 73.025) (end 183.2356 73.025) (width 0.2) (layer "F.Cu") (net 8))
 (segment (start 180.0935 71.353) (end 180.0935 70.603) (width 0.2) (layer "F.Cu") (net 8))
 (segment (start 180.8875 72.6835) (end 181.229 73.025) (width 0.2) (layer "F.Cu") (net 8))
 (segment (start 180.0935 71.375) (end 180.0935 71.353) (width 0.2) (layer "F.Cu") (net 8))
 (segment (start 183.2356 73.025) (end 181.706 73.025) (width 0.2) (layer "F.Cu") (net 8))
 (segment (start 181.229 73.025) (end 181.706 73.025) (width 0.2) (layer "F.Cu") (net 8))
 (segment (start 180.8875 72.644) (end 180.8875 72.6835) (width 0.2) (layer "F.Cu") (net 8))
 (segment (start 180.8875 72.169) (end 180.0935 71.375) (width 0.2) (layer "F.Cu") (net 8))
 (segment (start 180.8875 72.644) (end 180.8875 72.169) (width 0.2) (layer "F.Cu") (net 8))
 (segment (start 189.555 71.58) (end 185.722 71.58) (width 0.2) (layer "F.Cu") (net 8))
 (segment (start 179.4435 72.513) (end 179.3125 72.644) (width 0.2) (layer "F.Cu") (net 7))
 (segment (start 179.3125 72.644) (end 179.3125 73.7875) (width 0.2) (layer "F.Cu") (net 7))
 (segment (start 177.83556 73.8125) (end 177.8254 73.82266) (width 0.2) (layer "F.Cu") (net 7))
 (segment (start 179.4435 70.603) (end 179.4435 72.513) (width 0.2) (layer "F.Cu") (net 7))
 (segment (start 182.3974 73.8125) (end 179.3 73.8) (width 0.2) (layer "F.Cu") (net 7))
 (segment (start 179.3125 73.7875) (end 179.3 73.8) (width 0.2) (layer "F.Cu") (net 7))
 (segment (start 179.3 73.8) (end 177.83556 73.8125) (width 0.2) (layer "F.Cu") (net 7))
 (segment (start 179.36464 63.22568) (end 177.80508 63.22558) (width 0.2) (layer "F.Cu") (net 4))
 (segment (start 182.372 63.22558) (end 179.36464 63.22568) (width 0.2) (layer "F.Cu") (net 4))
 (segment (start 177.8001 63.2206) (end 177.8 63.2205) (width 0.25) (layer "F.Cu") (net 4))
 (segment (start 177.80508 63.22558) (end 177.8 63.2205) (width 0.2) (layer "F.Cu") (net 4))
 (segment (start 180.0935 65.1585) (end 180.0935 66.303) (width 0.2) (layer "F.Cu") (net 4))
 (segment (start 179.3125 63.27782) (end 179.3125 64.389) (width 0.2) (layer "F.Cu") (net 4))
 (segment (start 179.324 64.389) (end 180.0935 65.1585) (width 0.2) (layer "F.Cu") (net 4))
 (segment (start 179.3125 63.27782) (end 179.36464 63.22568) (width 0.2) (layer "F.Cu") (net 4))
 (segment (start 179.3125 64.389) (end 179.324 64.389) (width 0.2) (layer "F.Cu") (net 4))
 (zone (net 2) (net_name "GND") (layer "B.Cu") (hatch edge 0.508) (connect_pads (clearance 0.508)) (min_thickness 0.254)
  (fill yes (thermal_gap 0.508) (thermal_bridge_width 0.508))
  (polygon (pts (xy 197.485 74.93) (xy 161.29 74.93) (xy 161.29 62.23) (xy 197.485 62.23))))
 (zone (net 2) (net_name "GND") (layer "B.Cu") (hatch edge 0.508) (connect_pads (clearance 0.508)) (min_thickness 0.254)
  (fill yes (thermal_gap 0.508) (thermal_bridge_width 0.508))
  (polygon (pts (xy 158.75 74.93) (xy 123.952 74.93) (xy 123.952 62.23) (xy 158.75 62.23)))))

